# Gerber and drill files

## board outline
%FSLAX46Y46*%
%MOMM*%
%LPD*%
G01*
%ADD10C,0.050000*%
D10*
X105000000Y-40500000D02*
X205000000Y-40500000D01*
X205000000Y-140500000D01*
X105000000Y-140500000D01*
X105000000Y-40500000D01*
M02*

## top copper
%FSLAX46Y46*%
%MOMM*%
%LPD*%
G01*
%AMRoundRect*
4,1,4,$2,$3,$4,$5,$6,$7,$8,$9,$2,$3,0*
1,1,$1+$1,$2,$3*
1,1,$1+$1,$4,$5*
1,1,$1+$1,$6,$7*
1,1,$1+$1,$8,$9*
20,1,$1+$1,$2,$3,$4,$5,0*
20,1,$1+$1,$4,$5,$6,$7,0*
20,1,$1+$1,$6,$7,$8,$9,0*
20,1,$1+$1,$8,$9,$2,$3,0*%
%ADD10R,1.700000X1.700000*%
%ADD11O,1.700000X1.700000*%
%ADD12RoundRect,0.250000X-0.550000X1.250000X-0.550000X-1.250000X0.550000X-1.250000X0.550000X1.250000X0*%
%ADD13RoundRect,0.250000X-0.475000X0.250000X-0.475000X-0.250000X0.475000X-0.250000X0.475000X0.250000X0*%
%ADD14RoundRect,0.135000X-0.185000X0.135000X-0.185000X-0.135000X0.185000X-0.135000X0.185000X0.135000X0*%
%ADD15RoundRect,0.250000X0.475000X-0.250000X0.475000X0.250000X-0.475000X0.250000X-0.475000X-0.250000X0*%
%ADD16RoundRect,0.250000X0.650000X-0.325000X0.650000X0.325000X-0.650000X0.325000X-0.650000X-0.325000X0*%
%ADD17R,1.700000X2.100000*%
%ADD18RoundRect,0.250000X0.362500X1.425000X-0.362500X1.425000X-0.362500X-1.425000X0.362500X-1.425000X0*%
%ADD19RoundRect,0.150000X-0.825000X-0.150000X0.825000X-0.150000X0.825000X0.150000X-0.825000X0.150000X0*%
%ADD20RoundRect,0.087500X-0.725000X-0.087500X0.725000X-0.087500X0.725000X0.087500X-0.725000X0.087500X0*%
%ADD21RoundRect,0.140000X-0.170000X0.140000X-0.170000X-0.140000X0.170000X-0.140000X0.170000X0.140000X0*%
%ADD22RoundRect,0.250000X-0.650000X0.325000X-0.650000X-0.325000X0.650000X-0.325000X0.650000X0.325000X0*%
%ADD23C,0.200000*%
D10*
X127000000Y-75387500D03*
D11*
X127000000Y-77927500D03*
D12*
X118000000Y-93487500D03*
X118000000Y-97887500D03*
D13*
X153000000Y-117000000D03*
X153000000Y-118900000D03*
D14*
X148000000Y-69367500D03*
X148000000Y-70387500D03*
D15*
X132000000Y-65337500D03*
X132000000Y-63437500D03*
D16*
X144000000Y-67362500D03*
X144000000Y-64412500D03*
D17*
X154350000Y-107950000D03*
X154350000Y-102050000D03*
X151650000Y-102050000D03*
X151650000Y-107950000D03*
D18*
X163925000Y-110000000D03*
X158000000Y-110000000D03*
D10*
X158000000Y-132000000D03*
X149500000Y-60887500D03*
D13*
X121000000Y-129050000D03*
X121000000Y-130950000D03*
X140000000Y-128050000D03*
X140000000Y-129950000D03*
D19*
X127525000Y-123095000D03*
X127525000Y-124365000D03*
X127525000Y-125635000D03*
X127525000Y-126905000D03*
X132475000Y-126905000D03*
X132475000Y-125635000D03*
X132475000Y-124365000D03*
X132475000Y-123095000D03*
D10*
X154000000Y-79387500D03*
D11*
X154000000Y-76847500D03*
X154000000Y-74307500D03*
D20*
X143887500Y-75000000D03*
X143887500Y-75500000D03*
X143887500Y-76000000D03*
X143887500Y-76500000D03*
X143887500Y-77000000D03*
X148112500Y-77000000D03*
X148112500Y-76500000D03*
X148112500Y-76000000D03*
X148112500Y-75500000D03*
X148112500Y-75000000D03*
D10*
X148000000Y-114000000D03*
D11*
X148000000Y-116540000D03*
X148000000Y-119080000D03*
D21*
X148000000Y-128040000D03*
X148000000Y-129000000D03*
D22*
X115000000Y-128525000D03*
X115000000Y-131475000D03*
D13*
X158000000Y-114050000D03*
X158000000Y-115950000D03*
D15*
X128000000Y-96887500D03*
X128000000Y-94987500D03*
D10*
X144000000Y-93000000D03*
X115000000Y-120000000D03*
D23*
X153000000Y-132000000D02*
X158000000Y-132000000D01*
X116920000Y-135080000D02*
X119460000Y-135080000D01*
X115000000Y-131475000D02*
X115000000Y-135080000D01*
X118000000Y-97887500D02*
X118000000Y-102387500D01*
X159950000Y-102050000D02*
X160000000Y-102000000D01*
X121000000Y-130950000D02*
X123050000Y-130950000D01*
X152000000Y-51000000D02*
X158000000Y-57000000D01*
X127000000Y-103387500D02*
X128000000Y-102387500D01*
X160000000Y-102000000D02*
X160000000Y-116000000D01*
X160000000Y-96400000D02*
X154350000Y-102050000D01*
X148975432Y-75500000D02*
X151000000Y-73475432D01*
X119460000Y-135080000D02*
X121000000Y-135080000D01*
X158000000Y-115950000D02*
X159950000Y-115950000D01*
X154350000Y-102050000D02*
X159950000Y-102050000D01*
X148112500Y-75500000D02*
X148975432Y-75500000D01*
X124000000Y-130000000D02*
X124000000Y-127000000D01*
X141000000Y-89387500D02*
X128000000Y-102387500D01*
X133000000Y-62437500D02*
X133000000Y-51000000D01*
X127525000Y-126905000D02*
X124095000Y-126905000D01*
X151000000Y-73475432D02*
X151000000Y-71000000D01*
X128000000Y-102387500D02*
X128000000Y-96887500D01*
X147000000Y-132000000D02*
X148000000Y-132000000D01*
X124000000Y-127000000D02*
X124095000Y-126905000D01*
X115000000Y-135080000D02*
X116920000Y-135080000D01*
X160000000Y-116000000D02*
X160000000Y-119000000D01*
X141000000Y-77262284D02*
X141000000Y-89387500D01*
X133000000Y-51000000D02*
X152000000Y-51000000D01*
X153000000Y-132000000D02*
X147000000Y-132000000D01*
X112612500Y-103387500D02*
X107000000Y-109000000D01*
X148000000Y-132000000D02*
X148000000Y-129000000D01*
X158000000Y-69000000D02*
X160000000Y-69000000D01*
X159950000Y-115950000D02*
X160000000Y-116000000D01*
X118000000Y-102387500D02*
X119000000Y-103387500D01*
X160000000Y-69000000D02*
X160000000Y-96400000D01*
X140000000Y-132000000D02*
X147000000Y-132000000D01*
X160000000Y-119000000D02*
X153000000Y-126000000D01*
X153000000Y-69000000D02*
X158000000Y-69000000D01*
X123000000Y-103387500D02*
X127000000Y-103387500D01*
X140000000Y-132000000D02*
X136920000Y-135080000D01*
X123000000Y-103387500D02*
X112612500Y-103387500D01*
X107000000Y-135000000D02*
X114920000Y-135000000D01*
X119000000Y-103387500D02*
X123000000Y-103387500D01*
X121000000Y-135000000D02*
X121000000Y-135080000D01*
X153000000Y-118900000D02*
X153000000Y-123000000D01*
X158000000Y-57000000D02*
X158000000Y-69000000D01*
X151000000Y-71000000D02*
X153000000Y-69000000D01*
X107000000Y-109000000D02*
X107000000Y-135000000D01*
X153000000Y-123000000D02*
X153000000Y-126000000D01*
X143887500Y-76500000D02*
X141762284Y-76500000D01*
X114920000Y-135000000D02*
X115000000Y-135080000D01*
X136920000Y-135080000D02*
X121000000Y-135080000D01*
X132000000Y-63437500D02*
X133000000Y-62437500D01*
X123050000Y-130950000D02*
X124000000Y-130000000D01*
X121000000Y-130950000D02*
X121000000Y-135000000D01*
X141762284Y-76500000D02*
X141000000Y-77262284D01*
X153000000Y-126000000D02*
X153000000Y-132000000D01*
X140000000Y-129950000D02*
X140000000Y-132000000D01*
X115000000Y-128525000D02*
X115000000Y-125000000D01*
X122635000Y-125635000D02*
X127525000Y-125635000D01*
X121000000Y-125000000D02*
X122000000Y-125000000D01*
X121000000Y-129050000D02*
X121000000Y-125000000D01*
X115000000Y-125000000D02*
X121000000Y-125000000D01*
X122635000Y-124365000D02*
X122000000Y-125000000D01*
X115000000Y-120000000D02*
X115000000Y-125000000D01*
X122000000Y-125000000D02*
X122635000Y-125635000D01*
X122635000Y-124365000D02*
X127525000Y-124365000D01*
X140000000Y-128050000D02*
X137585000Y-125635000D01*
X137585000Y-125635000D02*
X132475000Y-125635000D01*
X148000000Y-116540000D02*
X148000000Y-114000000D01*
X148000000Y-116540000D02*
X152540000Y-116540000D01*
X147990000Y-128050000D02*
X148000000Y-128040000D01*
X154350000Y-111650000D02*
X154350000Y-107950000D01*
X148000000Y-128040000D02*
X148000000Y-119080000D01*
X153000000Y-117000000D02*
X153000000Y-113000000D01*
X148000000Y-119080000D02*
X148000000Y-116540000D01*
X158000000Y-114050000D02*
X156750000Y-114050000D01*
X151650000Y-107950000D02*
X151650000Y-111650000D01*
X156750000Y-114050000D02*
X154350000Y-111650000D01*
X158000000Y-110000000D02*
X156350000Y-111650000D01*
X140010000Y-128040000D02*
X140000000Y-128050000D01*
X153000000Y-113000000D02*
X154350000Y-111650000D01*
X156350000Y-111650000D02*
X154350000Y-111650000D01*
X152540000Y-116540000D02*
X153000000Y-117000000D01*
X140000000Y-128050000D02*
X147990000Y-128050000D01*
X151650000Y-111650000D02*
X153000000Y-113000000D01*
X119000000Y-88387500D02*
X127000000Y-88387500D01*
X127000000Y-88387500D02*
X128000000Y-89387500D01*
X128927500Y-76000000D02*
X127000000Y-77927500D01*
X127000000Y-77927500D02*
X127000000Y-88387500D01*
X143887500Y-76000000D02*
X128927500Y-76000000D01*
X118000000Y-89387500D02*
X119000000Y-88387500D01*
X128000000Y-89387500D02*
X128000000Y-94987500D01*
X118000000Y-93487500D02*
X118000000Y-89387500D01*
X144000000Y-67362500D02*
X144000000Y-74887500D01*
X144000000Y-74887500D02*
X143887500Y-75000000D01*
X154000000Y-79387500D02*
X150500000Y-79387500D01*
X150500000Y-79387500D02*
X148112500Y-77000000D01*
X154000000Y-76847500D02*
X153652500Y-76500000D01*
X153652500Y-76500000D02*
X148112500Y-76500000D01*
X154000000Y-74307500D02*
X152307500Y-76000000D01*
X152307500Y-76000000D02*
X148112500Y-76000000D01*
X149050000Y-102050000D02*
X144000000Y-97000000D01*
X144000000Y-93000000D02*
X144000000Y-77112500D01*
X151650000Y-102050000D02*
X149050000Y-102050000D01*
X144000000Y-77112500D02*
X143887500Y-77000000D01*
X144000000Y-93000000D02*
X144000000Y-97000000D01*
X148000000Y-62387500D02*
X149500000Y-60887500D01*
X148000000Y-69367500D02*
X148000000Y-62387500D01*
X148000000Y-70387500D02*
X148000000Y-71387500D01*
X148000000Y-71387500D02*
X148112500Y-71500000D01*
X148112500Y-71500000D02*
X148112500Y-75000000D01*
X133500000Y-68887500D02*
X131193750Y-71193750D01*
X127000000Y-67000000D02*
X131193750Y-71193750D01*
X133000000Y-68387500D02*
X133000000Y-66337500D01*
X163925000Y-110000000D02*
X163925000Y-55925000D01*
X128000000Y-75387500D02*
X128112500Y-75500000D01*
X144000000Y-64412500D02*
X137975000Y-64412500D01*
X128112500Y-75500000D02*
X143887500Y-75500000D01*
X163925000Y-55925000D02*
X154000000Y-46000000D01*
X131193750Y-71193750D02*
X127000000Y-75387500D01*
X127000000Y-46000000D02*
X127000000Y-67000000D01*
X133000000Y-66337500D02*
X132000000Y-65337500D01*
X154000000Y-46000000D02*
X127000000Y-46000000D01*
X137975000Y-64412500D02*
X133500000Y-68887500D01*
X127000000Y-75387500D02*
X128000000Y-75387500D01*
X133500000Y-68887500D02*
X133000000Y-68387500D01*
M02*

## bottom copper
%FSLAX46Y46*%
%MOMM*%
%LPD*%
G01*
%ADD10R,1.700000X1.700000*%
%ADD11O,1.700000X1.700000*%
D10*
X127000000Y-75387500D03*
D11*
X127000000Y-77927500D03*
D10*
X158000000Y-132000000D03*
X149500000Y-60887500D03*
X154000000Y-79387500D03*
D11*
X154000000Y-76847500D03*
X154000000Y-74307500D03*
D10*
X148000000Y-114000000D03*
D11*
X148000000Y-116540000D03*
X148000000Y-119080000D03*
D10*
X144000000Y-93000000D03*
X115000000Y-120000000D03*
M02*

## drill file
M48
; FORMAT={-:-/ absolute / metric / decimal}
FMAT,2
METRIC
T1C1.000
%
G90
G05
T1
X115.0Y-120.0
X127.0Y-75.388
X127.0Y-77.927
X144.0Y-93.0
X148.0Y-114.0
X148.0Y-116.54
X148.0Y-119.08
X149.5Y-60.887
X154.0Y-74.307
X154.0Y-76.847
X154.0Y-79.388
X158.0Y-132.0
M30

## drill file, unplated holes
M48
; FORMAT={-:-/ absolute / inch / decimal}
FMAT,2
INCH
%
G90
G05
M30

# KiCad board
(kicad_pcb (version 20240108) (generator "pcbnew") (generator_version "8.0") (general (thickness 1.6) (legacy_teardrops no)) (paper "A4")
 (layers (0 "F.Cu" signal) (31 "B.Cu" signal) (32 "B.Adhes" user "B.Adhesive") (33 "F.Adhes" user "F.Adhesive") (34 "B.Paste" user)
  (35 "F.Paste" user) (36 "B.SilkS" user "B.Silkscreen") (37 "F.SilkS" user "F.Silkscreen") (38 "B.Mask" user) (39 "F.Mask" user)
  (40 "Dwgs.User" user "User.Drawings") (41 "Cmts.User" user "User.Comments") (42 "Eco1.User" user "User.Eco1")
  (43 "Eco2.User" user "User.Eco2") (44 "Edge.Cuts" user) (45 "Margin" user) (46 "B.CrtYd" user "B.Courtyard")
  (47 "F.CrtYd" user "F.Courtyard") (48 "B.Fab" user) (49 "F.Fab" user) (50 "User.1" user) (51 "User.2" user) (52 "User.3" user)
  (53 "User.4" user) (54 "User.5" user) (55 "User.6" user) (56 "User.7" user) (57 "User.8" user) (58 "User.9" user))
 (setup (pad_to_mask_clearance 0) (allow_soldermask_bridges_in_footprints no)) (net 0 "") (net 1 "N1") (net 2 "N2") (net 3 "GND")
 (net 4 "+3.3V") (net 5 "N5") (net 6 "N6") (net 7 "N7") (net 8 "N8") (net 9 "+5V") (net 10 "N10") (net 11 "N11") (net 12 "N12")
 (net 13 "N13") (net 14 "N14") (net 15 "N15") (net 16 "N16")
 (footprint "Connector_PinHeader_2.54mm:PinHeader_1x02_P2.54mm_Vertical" (layer "F.Cu") (at 127 75.3875)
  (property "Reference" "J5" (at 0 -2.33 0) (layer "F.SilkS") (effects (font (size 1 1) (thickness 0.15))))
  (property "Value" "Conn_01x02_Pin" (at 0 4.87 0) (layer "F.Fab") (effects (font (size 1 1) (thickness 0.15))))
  (pad "1" thru_hole rect (at 0 0) (size 1.7 1.7) (drill 1) (layers "*.Cu" "*.Mask") (remove_unused_layers no) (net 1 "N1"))
  (pad "2" thru_hole oval (at 0 2.54) (size 1.7 1.7) (drill 1) (layers "*.Cu" "*.Mask") (remove_unused_layers no) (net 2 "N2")))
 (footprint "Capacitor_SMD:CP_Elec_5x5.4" (layer "F.Cu") (at 118 95.6875 -90)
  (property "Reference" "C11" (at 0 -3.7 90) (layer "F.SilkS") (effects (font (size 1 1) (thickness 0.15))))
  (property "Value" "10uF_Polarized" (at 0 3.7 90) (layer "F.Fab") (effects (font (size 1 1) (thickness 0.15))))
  (pad "1" smd roundrect (at -2.2 0 270) (size 3 1.6) (layers "F.Cu" "F.Paste" "F.Mask") (roundrect_rratio 0.15625) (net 2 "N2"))
  (pad "2" smd roundrect (at 2.2 0 270) (size 3 1.6) (layers "F.Cu" "F.Paste" "F.Mask") (roundrect_rratio 0.15625) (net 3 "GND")))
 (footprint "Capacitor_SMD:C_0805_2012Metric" (layer "F.Cu") (at 153 117.95 -90)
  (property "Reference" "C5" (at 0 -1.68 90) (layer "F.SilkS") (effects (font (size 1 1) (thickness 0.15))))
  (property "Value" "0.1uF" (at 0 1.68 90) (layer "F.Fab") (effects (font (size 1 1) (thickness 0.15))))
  (pad "1" smd roundrect (at -0.95 0 270) (size 1 1.45) (layers "F.Cu" "F.Paste" "F.Mask") (roundrect_rratio 0.25) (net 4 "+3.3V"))
  (pad "2" smd roundrect (at 0.95 0 270) (size 1 1.45) (layers "F.Cu" "F.Paste" "F.Mask") (roundrect_rratio 0.25) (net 3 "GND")))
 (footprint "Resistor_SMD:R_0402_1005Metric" (layer "F.Cu") (at 148 69.8775 -90)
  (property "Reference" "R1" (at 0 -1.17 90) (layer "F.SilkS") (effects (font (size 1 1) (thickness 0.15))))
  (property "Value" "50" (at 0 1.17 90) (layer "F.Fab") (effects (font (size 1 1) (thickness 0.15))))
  (pad "1" smd roundrect (at -0.51 0 270) (size 0.54 0.64) (layers "F.Cu" "F.Paste" "F.Mask") (roundrect_rratio 0.25) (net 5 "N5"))
  (pad "2" smd roundrect (at 0.51 0 270) (size 0.54 0.64) (layers "F.Cu" "F.Paste" "F.Mask") (roundrect_rratio 0.25) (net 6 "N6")))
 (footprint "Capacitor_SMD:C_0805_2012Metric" (layer "F.Cu") (at 132 64.3875 90)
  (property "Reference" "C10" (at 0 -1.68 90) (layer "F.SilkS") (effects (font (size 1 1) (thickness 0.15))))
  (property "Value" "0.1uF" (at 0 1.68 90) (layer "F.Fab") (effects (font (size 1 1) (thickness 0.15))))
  (pad "1" smd roundrect (at -0.95 0 90) (size 1 1.45) (layers "F.Cu" "F.Paste" "F.Mask") (roundrect_rratio 0.25) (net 1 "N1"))
  (pad "2" smd roundrect (at 0.95 0 90) (size 1 1.45) (layers "F.Cu" "F.Paste" "F.Mask") (roundrect_rratio 0.25) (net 3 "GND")))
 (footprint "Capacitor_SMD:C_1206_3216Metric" (layer "F.Cu") (at 144 65.8875 90)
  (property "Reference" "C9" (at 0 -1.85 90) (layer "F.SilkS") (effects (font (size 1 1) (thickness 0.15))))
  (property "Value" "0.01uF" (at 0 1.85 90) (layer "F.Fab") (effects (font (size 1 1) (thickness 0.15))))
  (pad "1" smd roundrect (at -1.475 0 90) (size 1.15 1.8) (layers "F.Cu" "F.Paste" "F.Mask") (roundrect_rratio 0.217391) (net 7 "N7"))
  (pad "2" smd roundrect (at 1.475 0 90) (size 1.15 1.8) (layers "F.Cu" "F.Paste" "F.Mask") (roundrect_rratio 0.217391) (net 1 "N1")))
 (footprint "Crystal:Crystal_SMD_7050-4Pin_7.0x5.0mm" (layer "F.Cu") (at 153 105 90)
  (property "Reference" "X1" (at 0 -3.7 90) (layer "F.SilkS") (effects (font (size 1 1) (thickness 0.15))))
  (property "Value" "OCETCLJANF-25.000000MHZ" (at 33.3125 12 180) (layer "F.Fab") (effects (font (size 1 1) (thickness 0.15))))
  (pad "1" smd rect (at -2.95 1.35 90) (size 2.1 1.7) (layers "F.Cu" "F.Paste" "F.Mask") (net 4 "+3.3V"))
  (pad "2" smd rect (at 2.95 1.35 90) (size 2.1 1.7) (layers "F.Cu" "F.Paste" "F.Mask") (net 3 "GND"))
  (pad "3" smd rect (at 2.95 -1.35 90) (size 2.1 1.7) (layers "F.Cu" "F.Paste" "F.Mask") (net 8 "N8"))
  (pad "4" smd rect (at -2.95 -1.35 90) (size 2.1 1.7) (layers "F.Cu" "F.Paste" "F.Mask") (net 4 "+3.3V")))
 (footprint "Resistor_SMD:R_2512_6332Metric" (layer "F.Cu") (at 160.9625 110 180)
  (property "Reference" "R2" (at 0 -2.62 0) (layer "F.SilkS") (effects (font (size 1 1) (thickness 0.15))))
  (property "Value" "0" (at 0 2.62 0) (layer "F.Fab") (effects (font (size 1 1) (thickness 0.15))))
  (pad "1" smd roundrect (at -2.9625 0 180) (size 1.225 3.35) (layers "F.Cu" "F.Paste" "F.Mask") (roundrect_rratio 0.204082) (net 1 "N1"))
  (pad "2" smd roundrect (at 2.9625 0 180) (size 1.225 3.35) (layers "F.Cu" "F.Paste" "F.Mask") (roundrect_rratio 0.204082) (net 4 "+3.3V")))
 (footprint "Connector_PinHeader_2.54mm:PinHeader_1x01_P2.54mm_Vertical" (layer "F.Cu") (at 158 132)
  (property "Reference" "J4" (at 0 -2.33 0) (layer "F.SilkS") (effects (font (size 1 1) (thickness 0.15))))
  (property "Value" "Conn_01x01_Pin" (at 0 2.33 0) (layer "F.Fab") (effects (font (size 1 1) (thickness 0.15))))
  (pad "1" thru_hole rect (at 0 0) (size 1.7 1.7) (drill 1) (layers "*.Cu" "*.Mask") (remove_unused_layers no) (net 3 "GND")))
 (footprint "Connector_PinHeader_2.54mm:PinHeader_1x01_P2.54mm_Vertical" (layer "F.Cu") (at 149.5 60.8875 90)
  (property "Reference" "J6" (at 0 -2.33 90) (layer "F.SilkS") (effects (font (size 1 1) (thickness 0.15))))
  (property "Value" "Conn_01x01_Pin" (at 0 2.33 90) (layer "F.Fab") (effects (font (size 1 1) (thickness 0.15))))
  (pad "1" thru_hole rect (at 0 0 90) (size 1.7 1.7) (drill 1) (layers "*.Cu" "*.Mask") (remove_unused_layers no) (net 5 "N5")))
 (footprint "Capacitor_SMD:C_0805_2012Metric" (layer "F.Cu") (at 121 130 -90)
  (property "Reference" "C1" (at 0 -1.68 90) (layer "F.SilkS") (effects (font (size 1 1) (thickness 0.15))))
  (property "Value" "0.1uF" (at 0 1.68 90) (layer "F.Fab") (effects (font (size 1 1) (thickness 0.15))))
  (pad "1" smd roundrect (at -0.95 0 270) (size 1 1.45) (layers "F.Cu" "F.Paste" "F.Mask") (roundrect_rratio 0.25) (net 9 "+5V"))
  (pad "2" smd roundrect (at 0.95 0 270) (size 1 1.45) (layers "F.Cu" "F.Paste" "F.Mask") (roundrect_rratio 0.25) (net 3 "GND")))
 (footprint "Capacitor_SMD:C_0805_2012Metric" (layer "F.Cu") (at 140 129 -90)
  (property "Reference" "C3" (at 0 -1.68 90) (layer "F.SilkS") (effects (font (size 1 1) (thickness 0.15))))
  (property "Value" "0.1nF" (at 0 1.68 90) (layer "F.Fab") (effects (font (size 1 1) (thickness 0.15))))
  (pad "1" smd roundrect (at -0.95 0 270) (size 1 1.45) (layers "F.Cu" "F.Paste" "F.Mask") (roundrect_rratio 0.25) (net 4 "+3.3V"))
  (pad "2" smd roundrect (at 0.95 0 270) (size 1 1.45) (layers "F.Cu" "F.Paste" "F.Mask") (roundrect_rratio 0.25) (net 3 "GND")))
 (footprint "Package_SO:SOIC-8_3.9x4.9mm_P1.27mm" (layer "F.Cu") (at 130 125)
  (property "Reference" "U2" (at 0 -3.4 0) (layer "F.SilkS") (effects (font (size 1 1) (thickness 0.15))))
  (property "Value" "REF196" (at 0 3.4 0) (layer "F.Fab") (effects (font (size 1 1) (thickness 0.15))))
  (pad "1" smd roundrect (at -2.475 -1.905) (size 1.95 0.6) (layers "F.Cu" "F.Paste" "F.Mask") (roundrect_rratio 0.25) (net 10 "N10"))
  (pad "2" smd roundrect (at -2.475 -0.635) (size 1.95 0.6) (layers "F.Cu" "F.Paste" "F.Mask") (roundrect_rratio 0.25) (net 9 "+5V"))
  (pad "3" smd roundrect (at -2.475 0.635) (size 1.95 0.6) (layers "F.Cu" "F.Paste" "F.Mask") (roundrect_rratio 0.25) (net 9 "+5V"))
  (pad "4" smd roundrect (at -2.475 1.905) (size 1.95 0.6) (layers "F.Cu" "F.Paste" "F.Mask") (roundrect_rratio 0.25) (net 3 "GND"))
  (pad "5" smd roundrect (at 2.475 1.905) (size 1.95 0.6) (layers "F.Cu" "F.Paste" "F.Mask") (roundrect_rratio 0.25) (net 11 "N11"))
  (pad "6" smd roundrect (at 2.475 0.635) (size 1.95 0.6) (layers "F.Cu" "F.Paste" "F.Mask") (roundrect_rratio 0.25) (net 4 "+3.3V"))
  (pad "7" smd roundrect (at 2.475 -0.635) (size 1.95 0.6) (layers "F.Cu" "F.Paste" "F.Mask") (roundrect_rratio 0.25) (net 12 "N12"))
  (pad "8" smd roundrect (at 2.475 -1.905) (size 1.95 0.6) (layers "F.Cu" "F.Paste" "F.Mask") (roundrect_rratio 0.25) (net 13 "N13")))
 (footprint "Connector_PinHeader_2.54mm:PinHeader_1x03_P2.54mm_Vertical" (layer "F.Cu") (at 154 79.3875 180)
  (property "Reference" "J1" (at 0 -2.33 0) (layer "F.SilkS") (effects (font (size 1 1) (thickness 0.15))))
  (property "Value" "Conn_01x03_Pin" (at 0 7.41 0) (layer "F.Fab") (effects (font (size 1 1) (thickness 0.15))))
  (pad "1" thru_hole rect (at 0 0 180) (size 1.7 1.7) (drill 1) (layers "*.Cu" "*.Mask") (remove_unused_layers no) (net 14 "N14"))
  (pad "2" thru_hole oval (at 0 2.54 180) (size 1.7 1.7) (drill 1) (layers "*.Cu" "*.Mask") (remove_unused_layers no) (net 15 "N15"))
  (pad "3" thru_hole oval (at 0 5.08 180) (size 1.7 1.7) (drill 1) (layers "*.Cu" "*.Mask") (remove_unused_layers no) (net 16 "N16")))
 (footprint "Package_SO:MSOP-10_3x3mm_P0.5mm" (layer "F.Cu") (at 146 76)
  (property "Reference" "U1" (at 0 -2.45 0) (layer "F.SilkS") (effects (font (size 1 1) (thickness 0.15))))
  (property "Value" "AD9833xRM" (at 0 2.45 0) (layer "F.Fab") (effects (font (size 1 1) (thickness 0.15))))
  (pad "1" smd roundrect (at -2.1125 -1) (size 1.625 0.35) (layers "F.Cu" "F.Paste" "F.Mask") (roundrect_rratio 0.25) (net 7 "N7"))
  (pad "2" smd roundrect (at -2.1125 -0.5) (size 1.625 0.35) (layers "F.Cu" "F.Paste" "F.Mask") (roundrect_rratio 0.25) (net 1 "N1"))
  (pad "3" smd roundrect (at -2.1125 0) (size 1.625 0.35) (layers "F.Cu" "F.Paste" "F.Mask") (roundrect_rratio 0.25) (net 2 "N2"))
  (pad "4" smd roundrect (at -2.1125 0.5) (size 1.625 0.35) (layers "F.Cu" "F.Paste" "F.Mask") (roundrect_rratio 0.25) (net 3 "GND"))
  (pad "5" smd roundrect (at -2.1125 1) (size 1.625 0.35) (layers "F.Cu" "F.Paste" "F.Mask") (roundrect_rratio 0.25) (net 8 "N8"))
  (pad "6" smd roundrect (at 2.1125 1) (size 1.625 0.35) (layers "F.Cu" "F.Paste" "F.Mask") (roundrect_rratio 0.25) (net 14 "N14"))
  (pad "7" smd roundrect (at 2.1125 0.5) (size 1.625 0.35) (layers "F.Cu" "F.Paste" "F.Mask") (roundrect_rratio 0.25) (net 15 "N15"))
  (pad "8" smd roundrect (at 2.1125 0) (size 1.625 0.35) (layers "F.Cu" "F.Paste" "F.Mask") (roundrect_rratio 0.25) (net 16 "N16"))
  (pad "9" smd roundrect (at 2.1125 -0.5) (size 1.625 0.35) (layers "F.Cu" "F.Paste" "F.Mask") (roundrect_rratio 0.25) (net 3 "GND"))
  (pad "10" smd roundrect (at 2.1125 -1) (size 1.625 0.35) (layers "F.Cu" "F.Paste" "F.Mask") (roundrect_rratio 0.25) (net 6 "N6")))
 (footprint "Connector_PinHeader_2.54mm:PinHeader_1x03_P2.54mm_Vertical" (layer "F.Cu") (at 148 114)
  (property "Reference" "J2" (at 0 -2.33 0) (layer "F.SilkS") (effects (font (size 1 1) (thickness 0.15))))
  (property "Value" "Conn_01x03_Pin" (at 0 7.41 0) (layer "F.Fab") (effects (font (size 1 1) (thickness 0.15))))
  (pad "1" thru_hole rect (at 0 0) (size 1.7 1.7) (drill 1) (layers "*.Cu" "*.Mask") (remove_unused_layers no) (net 4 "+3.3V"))
  (pad "2" thru_hole oval (at 0 2.54) (size 1.7 1.7) (drill 1) (layers "*.Cu" "*.Mask") (remove_unused_layers no) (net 4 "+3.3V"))
  (pad "3" thru_hole oval (at 0 5.08) (size 1.7 1.7) (drill 1) (layers "*.Cu" "*.Mask") (remove_unused_layers no) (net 4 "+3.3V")))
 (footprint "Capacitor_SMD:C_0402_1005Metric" (layer "F.Cu") (at 148 128.52 -90)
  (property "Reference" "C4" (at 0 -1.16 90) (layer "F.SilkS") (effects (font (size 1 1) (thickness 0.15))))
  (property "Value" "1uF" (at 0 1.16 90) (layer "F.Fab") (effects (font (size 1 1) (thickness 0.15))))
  (pad "1" smd roundrect (at -0.48 0 270) (size 0.56 0.62) (layers "F.Cu" "F.Paste" "F.Mask") (roundrect_rratio 0.25) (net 4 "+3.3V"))
  (pad "2" smd roundrect (at 0.48 0 270) (size 0.56 0.62) (layers "F.Cu" "F.Paste" "F.Mask") (roundrect_rratio 0.25) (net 3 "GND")))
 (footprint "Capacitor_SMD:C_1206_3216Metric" (layer "F.Cu") (at 115 130 -90)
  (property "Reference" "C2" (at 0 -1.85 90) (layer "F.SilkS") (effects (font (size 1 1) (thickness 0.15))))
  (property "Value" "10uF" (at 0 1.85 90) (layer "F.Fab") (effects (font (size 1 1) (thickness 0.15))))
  (pad "1" smd roundrect (at -1.475 0 270) (size 1.15 1.8) (layers "F.Cu" "F.Paste" "F.Mask") (roundrect_rratio 0.217391) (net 9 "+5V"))
  (pad "2" smd roundrect (at 1.475 0 270) (size 1.15 1.8) (layers "F.Cu" "F.Paste" "F.Mask") (roundrect_rratio 0.217391) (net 3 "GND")))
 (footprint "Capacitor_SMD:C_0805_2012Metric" (layer "F.Cu") (at 158 115 -90)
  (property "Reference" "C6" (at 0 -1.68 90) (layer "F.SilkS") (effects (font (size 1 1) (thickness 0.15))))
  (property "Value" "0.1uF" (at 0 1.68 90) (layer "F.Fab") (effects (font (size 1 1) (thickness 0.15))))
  (pad "1" smd roundrect (at -0.95 0 270) (size 1 1.45) (layers "F.Cu" "F.Paste" "F.Mask") (roundrect_rratio 0.25) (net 4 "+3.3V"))
  (pad "2" smd roundrect (at 0.95 0 270) (size 1 1.45) (layers "F.Cu" "F.Paste" "F.Mask") (roundrect_rratio 0.25) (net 3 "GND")))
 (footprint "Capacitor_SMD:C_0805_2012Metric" (layer "F.Cu") (at 128 95.9375 90)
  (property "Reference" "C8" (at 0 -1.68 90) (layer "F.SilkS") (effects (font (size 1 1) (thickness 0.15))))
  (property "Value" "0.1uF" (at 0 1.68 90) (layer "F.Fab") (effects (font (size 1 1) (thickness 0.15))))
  (pad "1" smd roundrect (at -0.95 0 90) (size 1 1.45) (layers "F.Cu" "F.Paste" "F.Mask") (roundrect_rratio 0.25) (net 3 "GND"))
  (pad "2" smd roundrect (at 0.95 0 90) (size 1 1.45) (layers "F.Cu" "F.Paste" "F.Mask") (roundrect_rratio 0.25) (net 2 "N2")))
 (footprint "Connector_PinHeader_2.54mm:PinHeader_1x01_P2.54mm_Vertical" (layer "F.Cu") (at 144 93)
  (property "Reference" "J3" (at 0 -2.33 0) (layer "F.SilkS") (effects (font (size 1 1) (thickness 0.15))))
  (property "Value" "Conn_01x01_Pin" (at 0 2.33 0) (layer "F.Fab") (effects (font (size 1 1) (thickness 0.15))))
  (pad "1" thru_hole rect (at 0 0) (size 1.7 1.7) (drill 1) (layers "*.Cu" "*.Mask") (remove_unused_layers no) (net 8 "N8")))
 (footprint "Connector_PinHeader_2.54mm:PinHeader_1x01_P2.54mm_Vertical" (layer "F.Cu") (at 115 120)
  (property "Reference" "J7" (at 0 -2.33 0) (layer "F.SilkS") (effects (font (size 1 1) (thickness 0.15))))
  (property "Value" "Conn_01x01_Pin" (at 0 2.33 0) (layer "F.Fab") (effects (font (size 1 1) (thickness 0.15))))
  (pad "1" thru_hole rect (at 0 0) (size 1.7 1.7) (drill 1) (layers "*.Cu" "*.Mask") (remove_unused_layers no) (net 9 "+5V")))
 (gr_rect (start 105 40.5) (end 205 140.5) (stroke (width 0.05) (type default)) (fill none) (layer "Edge.Cuts"))
 (segment (start 153 132) (end 158 132) (width 0.2) (layer "F.Cu") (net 3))
 (segment (start 116.92 135.08) (end 119.46 135.08) (width 0.2) (layer "F.Cu") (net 3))
 (segment (start 115 131.475) (end 115 135.08) (width 0.2) (layer "F.Cu") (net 3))
 (segment (start 118 97.8875) (end 118 102.3875) (width 0.2) (layer "F.Cu") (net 3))
 (segment (start 159.95 102.05) (end 160 102) (width 0.2) (layer "F.Cu") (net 3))
 (segment (start 121 130.95) (end 123.05 130.95) (width 0.2) (layer "F.Cu") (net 3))
 (segment (start 152 51) (end 158 57) (width 0.2) (layer "F.Cu") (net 3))
 (segment (start 127 103.3875) (end 128 102.3875) (width 0.2) (layer "F.Cu") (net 3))
 (segment (start 160 102) (end 160 116) (width 0.2) (layer "F.Cu") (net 3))
 (segment (start 160 96.4) (end 154.35 102.05) (width 0.2) (layer "F.Cu") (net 3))
 (segment (start 148.975432 75.5) (end 151 73.475432) (width 0.2) (layer "F.Cu") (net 3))
 (segment (start 119.46 135.08) (end 121 135.08) (width 0.2) (layer "F.Cu") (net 3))
 (segment (start 158 115.95) (end 159.95 115.95) (width 0.2) (layer "F.Cu") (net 3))
 (segment (start 154.35 102.05) (end 159.95 102.05) (width 0.2) (layer "F.Cu") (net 3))
 (segment (start 148.1125 75.5) (end 148.975432 75.5) (width 0.2) (layer "F.Cu") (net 3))
 (segment (start 124 130) (end 124 127) (width 0.2) (layer "F.Cu") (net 3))
 (segment (start 141 89.3875) (end 128 102.3875) (width 0.2) (layer "F.Cu") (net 3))
 (segment (start 133 62.4375) (end 133 51) (width 0.2) (layer "F.Cu") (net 3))
 (segment (start 127.525 126.905) (end 124.095 126.905) (width 0.2) (layer "F.Cu") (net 3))
 (segment (start 151 73.475432) (end 151 71) (width 0.2) (layer "F.Cu") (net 3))
 (segment (start 128 102.3875) (end 128 96.8875) (width 0.2) (layer "F.Cu") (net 3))
 (segment (start 147 132) (end 148 132) (width 0.2) (layer "F.Cu") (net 3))
 (segment (start 124 127) (end 124.095 126.905) (width 0.2) (layer "F.Cu") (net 3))
 (segment (start 115 135.08) (end 116.92 135.08) (width 0.2) (layer "F.Cu") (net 3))
 (segment (start 160 116) (end 160 119) (width 0.2) (layer "F.Cu") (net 3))
 (segment (start 141 77.262284) (end 141 89.3875) (width 0.2) (layer "F.Cu") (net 3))
 (segment (start 133 51) (end 152 51) (width 0.2) (layer "F.Cu") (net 3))
 (segment (start 153 132) (end 147 132) (width 0.2) (layer "F.Cu") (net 3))
 (segment (start 112.6125 103.3875) (end 107 109) (width 0.2) (layer "F.Cu") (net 3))
 (segment (start 148 132) (end 148 129) (width 0.2) (layer "F.Cu") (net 3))
 (segment (start 158 69) (end 160 69) (width 0.2) (layer "F.Cu") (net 3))
 (segment (start 159.95 115.95) (end 160 116) (width 0.2) (layer "F.Cu") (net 3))
 (segment (start 118 102.3875) (end 119 103.3875) (width 0.2) (layer "F.Cu") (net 3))
 (segment (start 160 69) (end 160 96.4) (width 0.2) (layer "F.Cu") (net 3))
 (segment (start 140 132) (end 147 132) (width 0.2) (layer "F.Cu") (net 3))
 (segment (start 160 119) (end 153 126) (width 0.2) (layer "F.Cu") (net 3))
 (segment (start 153 69) (end 158 69) (width 0.2) (layer "F.Cu") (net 3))
 (segment (start 123 103.3875) (end 127 103.3875) (width 0.2) (layer "F.Cu") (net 3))
 (segment (start 140 132) (end 136.92 135.08) (width 0.2) (layer "F.Cu") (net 3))
 (segment (start 123 103.3875) (end 112.6125 103.3875) (width 0.2) (layer "F.Cu") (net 3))
 (segment (start 107 135) (end 114.92 135) (width 0.2) (layer "F.Cu") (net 3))
 (segment (start 119 103.3875) (end 123 103.3875) (width 0.2) (layer "F.Cu") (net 3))
 (segment (start 121 135) (end 121 135.08) (width 0.2) (layer "F.Cu") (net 3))
 (segment (start 153 118.9) (end 153 123) (width 0.2) (layer "F.Cu") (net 3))
 (segment (start 158 57) (end 158 69) (width 0.2) (layer "F.Cu") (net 3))
 (segment (start 151 71) (end 153 69) (width 0.2) (layer "F.Cu") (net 3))
 (segment (start 107 109) (end 107 135) (width 0.2) (layer "F.Cu") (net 3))
 (segment (start 153 123) (end 153 126) (width 0.2) (layer "F.Cu") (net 3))
 (segment (start 143.8875 76.5) (end 141.762284 76.5) (width 0.2) (layer "F.Cu") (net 3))
 (segment (start 114.92 135) (end 115 135.08) (width 0.2) (layer "F.Cu") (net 3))
 (segment (start 136.92 135.08) (end 121 135.08) (width 0.2) (layer "F.Cu") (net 3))
 (segment (start 132 63.4375) (end 133 62.4375) (width 0.2) (layer "F.Cu") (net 3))
 (segment (start 123.05 130.95) (end 124 130) (width 0.2) (layer "F.Cu") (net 3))
 (segment (start 121 130.95) (end 121 135) (width 0.2) (layer "F.Cu") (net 3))
 (segment (start 141.762284 76.5) (end 141 77.262284) (width 0.2) (layer "F.Cu") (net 3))
 (segment (start 153 126) (end 153 132) (width 0.2) (layer "F.Cu") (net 3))
 (segment (start 140 129.95) (end 140 132) (width 0.2) (layer "F.Cu") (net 3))
 (segment (start 115 128.525) (end 115 125) (width 0.2) (layer "F.Cu") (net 9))
 (segment (start 122.635 125.635) (end 127.525 125.635) (width 0.2) (layer "F.Cu") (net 9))
 (segment (start 121 125) (end 122 125) (width 0.2) (layer "F.Cu") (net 9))
 (segment (start 121 129.05) (end 121 125) (width 0.2) (layer "F.Cu") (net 9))
 (segment (start 115 125) (end 121 125) (width 0.2) (layer "F.Cu") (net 9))
 (segment (start 122.635 124.365) (end 122 125) (width 0.2) (layer "F.Cu") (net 9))
 (segment (start 115 120) (end 115 125) (width 0.2) (layer "F.Cu") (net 9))
 (segment (start 122 125) (end 122.635 125.635) (width 0.2) (layer "F.Cu") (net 9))
 (segment (start 122.635 124.365) (end 127.525 124.365) (width 0.2) (layer "F.Cu") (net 9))
 (segment (start 140 128.05) (end 137.585 125.635) (width 0.2) (layer "F.Cu") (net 4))
 (segment (start 137.585 125.635) (end 132.475 125.635) (width 0.2) (layer "F.Cu") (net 4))
 (segment (start 148 116.54) (end 148 114) (width 0.2) (layer "F.Cu") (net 4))
 (segment (start 148 116.54) (end 152.54 116.54) (width 0.2) (layer "F.Cu") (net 4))
 (segment (start 147.99 128.05) (end 148 128.04) (width 0.2) (layer "F.Cu") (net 4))
 (segment (start 154.35 111.65) (end 154.35 107.95) (width 0.2) (layer "F.Cu") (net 4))
 (segment (start 148 128.04) (end 148 119.08) (width 0.2) (layer "F.Cu") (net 4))
 (segment (start 153 117) (end 153 113) (width 0.2) (layer "F.Cu") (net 4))
 (segment (start 148 119.08) (end 148 116.54) (width 0.2) (layer "F.Cu") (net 4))
 (segment (start 158 114.05) (end 156.75 114.05) (width 0.2) (layer "F.Cu") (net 4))
 (segment (start 151.65 107.95) (end 151.65 111.65) (width 0.2) (layer "F.Cu") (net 4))
 (segment (start 156.75 114.05) (end 154.35 111.65) (width 0.2) (layer "F.Cu") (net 4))
 (segment (start 158 110) (end 156.35 111.65) (width 0.2) (layer "F.Cu") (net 4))
 (segment (start 140.01 128.04) (end 140 128.05) (width 0.2) (layer "F.Cu") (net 4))
 (segment (start 153 113) (end 154.35 111.65) (width 0.2) (layer "F.Cu") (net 4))
 (segment (start 156.35 111.65) (end 154.35 111.65) (width 0.2) (layer "F.Cu") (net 4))
 (segment (start 152.54 116.54) (end 153 117) (width 0.2) (layer "F.Cu") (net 4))
 (segment (start 140 128.05) (end 147.99 128.05) (width 0.2) (layer "F.Cu") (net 4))
 (segment (start 151.65 111.65) (end 153 113) (width 0.2) (layer "F.Cu") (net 4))
 (segment (start 119 88.3875) (end 127 88.3875) (width 0.2) (layer "F.Cu") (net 2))
 (segment (start 127 88.3875) (end 128 89.3875) (width 0.2) (layer "F.Cu") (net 2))
 (segment (start 128.9275 76) (end 127 77.9275) (width 0.2) (layer "F.Cu") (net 2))
 (segment (start 127 77.9275) (end 127 88.3875) (width 0.2) (layer "F.Cu") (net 2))
 (segment (start 143.8875 76) (end 128.9275 76) (width 0.2) (layer "F.Cu") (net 2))
 (segment (start 118 89.3875) (end 119 88.3875) (width 0.2) (layer "F.Cu") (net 2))
 (segment (start 128 89.3875) (end 128 94.9875) (width 0.2) (layer "F.Cu") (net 2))
 (segment (start 118 93.4875) (end 118 89.3875) (width 0.2) (layer "F.Cu") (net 2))
 (segment (start 144 67.3625) (end 144 74.8875) (width 0.2) (layer "F.Cu") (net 7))
 (segment (start 144 74.8875) (end 143.8875 75) (width 0.2) (layer "F.Cu") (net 7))
 (segment (start 154 79.3875) (end 150.5 79.3875) (width 0.2) (layer "F.Cu") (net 14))
 (segment (start 150.5 79.3875) (end 148.1125 77) (width 0.2) (layer "F.Cu") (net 14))
 (segment (start 154 76.8475) (end 153.6525 76.5) (width 0.2) (layer "F.Cu") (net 15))
 (segment (start 153.6525 76.5) (end 148.1125 76.5) (width 0.2) (layer "F.Cu") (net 15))
 (segment (start 154 74.3075) (end 152.3075 76) (width 0.2) (layer "F.Cu") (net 16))
 (segment (start 152.3075 76) (end 148.1125 76) (width 0.2) (layer "F.Cu") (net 16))
 (segment (start 149.05 102.05) (end 144 97) (width 0.2) (layer "F.Cu") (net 8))
 (segment (start 144 93) (end 144 77.1125) (width 0.2) (layer "F.Cu") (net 8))
 (segment (start 151.65 102.05) (end 149.05 102.05) (width 0.2) (layer "F.Cu") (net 8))
 (segment (start 144 77.1125) (end 143.8875 77) (width 0.2) (layer "F.Cu") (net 8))
 (segment (start 144 93) (end 144 97) (width 0.2) (layer "F.Cu") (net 8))
 (segment (start 148 62.3875) (end 149.5 60.8875) (width 0.2) (layer "F.Cu") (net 5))
 (segment (start 148 69.3675) (end 148 62.3875) (width 0.2) (layer "F.Cu") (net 5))
 (segment (start 148 70.3875) (end 148 71.3875) (width 0.2) (layer "F.Cu") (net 6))
 (segment (start 148 71.3875) (end 148.1125 71.5) (width 0.2) (layer "F.Cu") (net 6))
 (segment (start 148.1125 71.5) (end 148.1125 75) (width 0.2) (layer "F.Cu") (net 6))
 (segment (start 133.5 68.8875) (end 131.19375 71.19375) (width 0.2) (layer "F.Cu") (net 1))
 (segment (start 127 67) (end 131.19375 71.19375) (width 0.2) (layer "F.Cu") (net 1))
 (segment (start 133 68.3875) (end 133 66.3375) (width 0.2) (layer "F.Cu") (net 1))
 (segment (start 163.925 110) (end 163.925 55.925) (width 0.2) (layer "F.Cu") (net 1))
 (segment (start 128 75.3875) (end 128.1125 75.5) (width 0.2) (layer "F.Cu") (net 1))
 (segment (start 144 64.4125) (end 137.975 64.4125) (width 0.2) (layer "F.Cu") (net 1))
 (segment (start 128.1125 75.5) (end 143.8875 75.5) (width 0.2) (layer "F.Cu") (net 1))
 (segment (start 163.925 55.925) (end 154 46) (width 0.2) (layer "F.Cu") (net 1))
 (segment (start 131.19375 71.19375) (end 127 75.3875) (width 0.2) (layer "F.Cu") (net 1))
 (segment (start 127 46) (end 127 67) (width 0.2) (layer "F.Cu") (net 1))
 (segment (start 133 66.3375) (end 132 65.3375) (width 0.2) (layer "F.Cu") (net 1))
 (segment (start 154 46) (end 127 46) (width 0.2) (layer "F.Cu") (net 1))
 (segment (start 137.975 64.4125) (end 133.5 68.8875) (width 0.2) (layer "F.Cu") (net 1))
 (segment (start 127 75.3875) (end 128 75.3875) (width 0.2) (layer "F.Cu") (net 1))
 (segment (start 133.5 68.8875) (end 133 68.3875) (width 0.2) (layer "F.Cu") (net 1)))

